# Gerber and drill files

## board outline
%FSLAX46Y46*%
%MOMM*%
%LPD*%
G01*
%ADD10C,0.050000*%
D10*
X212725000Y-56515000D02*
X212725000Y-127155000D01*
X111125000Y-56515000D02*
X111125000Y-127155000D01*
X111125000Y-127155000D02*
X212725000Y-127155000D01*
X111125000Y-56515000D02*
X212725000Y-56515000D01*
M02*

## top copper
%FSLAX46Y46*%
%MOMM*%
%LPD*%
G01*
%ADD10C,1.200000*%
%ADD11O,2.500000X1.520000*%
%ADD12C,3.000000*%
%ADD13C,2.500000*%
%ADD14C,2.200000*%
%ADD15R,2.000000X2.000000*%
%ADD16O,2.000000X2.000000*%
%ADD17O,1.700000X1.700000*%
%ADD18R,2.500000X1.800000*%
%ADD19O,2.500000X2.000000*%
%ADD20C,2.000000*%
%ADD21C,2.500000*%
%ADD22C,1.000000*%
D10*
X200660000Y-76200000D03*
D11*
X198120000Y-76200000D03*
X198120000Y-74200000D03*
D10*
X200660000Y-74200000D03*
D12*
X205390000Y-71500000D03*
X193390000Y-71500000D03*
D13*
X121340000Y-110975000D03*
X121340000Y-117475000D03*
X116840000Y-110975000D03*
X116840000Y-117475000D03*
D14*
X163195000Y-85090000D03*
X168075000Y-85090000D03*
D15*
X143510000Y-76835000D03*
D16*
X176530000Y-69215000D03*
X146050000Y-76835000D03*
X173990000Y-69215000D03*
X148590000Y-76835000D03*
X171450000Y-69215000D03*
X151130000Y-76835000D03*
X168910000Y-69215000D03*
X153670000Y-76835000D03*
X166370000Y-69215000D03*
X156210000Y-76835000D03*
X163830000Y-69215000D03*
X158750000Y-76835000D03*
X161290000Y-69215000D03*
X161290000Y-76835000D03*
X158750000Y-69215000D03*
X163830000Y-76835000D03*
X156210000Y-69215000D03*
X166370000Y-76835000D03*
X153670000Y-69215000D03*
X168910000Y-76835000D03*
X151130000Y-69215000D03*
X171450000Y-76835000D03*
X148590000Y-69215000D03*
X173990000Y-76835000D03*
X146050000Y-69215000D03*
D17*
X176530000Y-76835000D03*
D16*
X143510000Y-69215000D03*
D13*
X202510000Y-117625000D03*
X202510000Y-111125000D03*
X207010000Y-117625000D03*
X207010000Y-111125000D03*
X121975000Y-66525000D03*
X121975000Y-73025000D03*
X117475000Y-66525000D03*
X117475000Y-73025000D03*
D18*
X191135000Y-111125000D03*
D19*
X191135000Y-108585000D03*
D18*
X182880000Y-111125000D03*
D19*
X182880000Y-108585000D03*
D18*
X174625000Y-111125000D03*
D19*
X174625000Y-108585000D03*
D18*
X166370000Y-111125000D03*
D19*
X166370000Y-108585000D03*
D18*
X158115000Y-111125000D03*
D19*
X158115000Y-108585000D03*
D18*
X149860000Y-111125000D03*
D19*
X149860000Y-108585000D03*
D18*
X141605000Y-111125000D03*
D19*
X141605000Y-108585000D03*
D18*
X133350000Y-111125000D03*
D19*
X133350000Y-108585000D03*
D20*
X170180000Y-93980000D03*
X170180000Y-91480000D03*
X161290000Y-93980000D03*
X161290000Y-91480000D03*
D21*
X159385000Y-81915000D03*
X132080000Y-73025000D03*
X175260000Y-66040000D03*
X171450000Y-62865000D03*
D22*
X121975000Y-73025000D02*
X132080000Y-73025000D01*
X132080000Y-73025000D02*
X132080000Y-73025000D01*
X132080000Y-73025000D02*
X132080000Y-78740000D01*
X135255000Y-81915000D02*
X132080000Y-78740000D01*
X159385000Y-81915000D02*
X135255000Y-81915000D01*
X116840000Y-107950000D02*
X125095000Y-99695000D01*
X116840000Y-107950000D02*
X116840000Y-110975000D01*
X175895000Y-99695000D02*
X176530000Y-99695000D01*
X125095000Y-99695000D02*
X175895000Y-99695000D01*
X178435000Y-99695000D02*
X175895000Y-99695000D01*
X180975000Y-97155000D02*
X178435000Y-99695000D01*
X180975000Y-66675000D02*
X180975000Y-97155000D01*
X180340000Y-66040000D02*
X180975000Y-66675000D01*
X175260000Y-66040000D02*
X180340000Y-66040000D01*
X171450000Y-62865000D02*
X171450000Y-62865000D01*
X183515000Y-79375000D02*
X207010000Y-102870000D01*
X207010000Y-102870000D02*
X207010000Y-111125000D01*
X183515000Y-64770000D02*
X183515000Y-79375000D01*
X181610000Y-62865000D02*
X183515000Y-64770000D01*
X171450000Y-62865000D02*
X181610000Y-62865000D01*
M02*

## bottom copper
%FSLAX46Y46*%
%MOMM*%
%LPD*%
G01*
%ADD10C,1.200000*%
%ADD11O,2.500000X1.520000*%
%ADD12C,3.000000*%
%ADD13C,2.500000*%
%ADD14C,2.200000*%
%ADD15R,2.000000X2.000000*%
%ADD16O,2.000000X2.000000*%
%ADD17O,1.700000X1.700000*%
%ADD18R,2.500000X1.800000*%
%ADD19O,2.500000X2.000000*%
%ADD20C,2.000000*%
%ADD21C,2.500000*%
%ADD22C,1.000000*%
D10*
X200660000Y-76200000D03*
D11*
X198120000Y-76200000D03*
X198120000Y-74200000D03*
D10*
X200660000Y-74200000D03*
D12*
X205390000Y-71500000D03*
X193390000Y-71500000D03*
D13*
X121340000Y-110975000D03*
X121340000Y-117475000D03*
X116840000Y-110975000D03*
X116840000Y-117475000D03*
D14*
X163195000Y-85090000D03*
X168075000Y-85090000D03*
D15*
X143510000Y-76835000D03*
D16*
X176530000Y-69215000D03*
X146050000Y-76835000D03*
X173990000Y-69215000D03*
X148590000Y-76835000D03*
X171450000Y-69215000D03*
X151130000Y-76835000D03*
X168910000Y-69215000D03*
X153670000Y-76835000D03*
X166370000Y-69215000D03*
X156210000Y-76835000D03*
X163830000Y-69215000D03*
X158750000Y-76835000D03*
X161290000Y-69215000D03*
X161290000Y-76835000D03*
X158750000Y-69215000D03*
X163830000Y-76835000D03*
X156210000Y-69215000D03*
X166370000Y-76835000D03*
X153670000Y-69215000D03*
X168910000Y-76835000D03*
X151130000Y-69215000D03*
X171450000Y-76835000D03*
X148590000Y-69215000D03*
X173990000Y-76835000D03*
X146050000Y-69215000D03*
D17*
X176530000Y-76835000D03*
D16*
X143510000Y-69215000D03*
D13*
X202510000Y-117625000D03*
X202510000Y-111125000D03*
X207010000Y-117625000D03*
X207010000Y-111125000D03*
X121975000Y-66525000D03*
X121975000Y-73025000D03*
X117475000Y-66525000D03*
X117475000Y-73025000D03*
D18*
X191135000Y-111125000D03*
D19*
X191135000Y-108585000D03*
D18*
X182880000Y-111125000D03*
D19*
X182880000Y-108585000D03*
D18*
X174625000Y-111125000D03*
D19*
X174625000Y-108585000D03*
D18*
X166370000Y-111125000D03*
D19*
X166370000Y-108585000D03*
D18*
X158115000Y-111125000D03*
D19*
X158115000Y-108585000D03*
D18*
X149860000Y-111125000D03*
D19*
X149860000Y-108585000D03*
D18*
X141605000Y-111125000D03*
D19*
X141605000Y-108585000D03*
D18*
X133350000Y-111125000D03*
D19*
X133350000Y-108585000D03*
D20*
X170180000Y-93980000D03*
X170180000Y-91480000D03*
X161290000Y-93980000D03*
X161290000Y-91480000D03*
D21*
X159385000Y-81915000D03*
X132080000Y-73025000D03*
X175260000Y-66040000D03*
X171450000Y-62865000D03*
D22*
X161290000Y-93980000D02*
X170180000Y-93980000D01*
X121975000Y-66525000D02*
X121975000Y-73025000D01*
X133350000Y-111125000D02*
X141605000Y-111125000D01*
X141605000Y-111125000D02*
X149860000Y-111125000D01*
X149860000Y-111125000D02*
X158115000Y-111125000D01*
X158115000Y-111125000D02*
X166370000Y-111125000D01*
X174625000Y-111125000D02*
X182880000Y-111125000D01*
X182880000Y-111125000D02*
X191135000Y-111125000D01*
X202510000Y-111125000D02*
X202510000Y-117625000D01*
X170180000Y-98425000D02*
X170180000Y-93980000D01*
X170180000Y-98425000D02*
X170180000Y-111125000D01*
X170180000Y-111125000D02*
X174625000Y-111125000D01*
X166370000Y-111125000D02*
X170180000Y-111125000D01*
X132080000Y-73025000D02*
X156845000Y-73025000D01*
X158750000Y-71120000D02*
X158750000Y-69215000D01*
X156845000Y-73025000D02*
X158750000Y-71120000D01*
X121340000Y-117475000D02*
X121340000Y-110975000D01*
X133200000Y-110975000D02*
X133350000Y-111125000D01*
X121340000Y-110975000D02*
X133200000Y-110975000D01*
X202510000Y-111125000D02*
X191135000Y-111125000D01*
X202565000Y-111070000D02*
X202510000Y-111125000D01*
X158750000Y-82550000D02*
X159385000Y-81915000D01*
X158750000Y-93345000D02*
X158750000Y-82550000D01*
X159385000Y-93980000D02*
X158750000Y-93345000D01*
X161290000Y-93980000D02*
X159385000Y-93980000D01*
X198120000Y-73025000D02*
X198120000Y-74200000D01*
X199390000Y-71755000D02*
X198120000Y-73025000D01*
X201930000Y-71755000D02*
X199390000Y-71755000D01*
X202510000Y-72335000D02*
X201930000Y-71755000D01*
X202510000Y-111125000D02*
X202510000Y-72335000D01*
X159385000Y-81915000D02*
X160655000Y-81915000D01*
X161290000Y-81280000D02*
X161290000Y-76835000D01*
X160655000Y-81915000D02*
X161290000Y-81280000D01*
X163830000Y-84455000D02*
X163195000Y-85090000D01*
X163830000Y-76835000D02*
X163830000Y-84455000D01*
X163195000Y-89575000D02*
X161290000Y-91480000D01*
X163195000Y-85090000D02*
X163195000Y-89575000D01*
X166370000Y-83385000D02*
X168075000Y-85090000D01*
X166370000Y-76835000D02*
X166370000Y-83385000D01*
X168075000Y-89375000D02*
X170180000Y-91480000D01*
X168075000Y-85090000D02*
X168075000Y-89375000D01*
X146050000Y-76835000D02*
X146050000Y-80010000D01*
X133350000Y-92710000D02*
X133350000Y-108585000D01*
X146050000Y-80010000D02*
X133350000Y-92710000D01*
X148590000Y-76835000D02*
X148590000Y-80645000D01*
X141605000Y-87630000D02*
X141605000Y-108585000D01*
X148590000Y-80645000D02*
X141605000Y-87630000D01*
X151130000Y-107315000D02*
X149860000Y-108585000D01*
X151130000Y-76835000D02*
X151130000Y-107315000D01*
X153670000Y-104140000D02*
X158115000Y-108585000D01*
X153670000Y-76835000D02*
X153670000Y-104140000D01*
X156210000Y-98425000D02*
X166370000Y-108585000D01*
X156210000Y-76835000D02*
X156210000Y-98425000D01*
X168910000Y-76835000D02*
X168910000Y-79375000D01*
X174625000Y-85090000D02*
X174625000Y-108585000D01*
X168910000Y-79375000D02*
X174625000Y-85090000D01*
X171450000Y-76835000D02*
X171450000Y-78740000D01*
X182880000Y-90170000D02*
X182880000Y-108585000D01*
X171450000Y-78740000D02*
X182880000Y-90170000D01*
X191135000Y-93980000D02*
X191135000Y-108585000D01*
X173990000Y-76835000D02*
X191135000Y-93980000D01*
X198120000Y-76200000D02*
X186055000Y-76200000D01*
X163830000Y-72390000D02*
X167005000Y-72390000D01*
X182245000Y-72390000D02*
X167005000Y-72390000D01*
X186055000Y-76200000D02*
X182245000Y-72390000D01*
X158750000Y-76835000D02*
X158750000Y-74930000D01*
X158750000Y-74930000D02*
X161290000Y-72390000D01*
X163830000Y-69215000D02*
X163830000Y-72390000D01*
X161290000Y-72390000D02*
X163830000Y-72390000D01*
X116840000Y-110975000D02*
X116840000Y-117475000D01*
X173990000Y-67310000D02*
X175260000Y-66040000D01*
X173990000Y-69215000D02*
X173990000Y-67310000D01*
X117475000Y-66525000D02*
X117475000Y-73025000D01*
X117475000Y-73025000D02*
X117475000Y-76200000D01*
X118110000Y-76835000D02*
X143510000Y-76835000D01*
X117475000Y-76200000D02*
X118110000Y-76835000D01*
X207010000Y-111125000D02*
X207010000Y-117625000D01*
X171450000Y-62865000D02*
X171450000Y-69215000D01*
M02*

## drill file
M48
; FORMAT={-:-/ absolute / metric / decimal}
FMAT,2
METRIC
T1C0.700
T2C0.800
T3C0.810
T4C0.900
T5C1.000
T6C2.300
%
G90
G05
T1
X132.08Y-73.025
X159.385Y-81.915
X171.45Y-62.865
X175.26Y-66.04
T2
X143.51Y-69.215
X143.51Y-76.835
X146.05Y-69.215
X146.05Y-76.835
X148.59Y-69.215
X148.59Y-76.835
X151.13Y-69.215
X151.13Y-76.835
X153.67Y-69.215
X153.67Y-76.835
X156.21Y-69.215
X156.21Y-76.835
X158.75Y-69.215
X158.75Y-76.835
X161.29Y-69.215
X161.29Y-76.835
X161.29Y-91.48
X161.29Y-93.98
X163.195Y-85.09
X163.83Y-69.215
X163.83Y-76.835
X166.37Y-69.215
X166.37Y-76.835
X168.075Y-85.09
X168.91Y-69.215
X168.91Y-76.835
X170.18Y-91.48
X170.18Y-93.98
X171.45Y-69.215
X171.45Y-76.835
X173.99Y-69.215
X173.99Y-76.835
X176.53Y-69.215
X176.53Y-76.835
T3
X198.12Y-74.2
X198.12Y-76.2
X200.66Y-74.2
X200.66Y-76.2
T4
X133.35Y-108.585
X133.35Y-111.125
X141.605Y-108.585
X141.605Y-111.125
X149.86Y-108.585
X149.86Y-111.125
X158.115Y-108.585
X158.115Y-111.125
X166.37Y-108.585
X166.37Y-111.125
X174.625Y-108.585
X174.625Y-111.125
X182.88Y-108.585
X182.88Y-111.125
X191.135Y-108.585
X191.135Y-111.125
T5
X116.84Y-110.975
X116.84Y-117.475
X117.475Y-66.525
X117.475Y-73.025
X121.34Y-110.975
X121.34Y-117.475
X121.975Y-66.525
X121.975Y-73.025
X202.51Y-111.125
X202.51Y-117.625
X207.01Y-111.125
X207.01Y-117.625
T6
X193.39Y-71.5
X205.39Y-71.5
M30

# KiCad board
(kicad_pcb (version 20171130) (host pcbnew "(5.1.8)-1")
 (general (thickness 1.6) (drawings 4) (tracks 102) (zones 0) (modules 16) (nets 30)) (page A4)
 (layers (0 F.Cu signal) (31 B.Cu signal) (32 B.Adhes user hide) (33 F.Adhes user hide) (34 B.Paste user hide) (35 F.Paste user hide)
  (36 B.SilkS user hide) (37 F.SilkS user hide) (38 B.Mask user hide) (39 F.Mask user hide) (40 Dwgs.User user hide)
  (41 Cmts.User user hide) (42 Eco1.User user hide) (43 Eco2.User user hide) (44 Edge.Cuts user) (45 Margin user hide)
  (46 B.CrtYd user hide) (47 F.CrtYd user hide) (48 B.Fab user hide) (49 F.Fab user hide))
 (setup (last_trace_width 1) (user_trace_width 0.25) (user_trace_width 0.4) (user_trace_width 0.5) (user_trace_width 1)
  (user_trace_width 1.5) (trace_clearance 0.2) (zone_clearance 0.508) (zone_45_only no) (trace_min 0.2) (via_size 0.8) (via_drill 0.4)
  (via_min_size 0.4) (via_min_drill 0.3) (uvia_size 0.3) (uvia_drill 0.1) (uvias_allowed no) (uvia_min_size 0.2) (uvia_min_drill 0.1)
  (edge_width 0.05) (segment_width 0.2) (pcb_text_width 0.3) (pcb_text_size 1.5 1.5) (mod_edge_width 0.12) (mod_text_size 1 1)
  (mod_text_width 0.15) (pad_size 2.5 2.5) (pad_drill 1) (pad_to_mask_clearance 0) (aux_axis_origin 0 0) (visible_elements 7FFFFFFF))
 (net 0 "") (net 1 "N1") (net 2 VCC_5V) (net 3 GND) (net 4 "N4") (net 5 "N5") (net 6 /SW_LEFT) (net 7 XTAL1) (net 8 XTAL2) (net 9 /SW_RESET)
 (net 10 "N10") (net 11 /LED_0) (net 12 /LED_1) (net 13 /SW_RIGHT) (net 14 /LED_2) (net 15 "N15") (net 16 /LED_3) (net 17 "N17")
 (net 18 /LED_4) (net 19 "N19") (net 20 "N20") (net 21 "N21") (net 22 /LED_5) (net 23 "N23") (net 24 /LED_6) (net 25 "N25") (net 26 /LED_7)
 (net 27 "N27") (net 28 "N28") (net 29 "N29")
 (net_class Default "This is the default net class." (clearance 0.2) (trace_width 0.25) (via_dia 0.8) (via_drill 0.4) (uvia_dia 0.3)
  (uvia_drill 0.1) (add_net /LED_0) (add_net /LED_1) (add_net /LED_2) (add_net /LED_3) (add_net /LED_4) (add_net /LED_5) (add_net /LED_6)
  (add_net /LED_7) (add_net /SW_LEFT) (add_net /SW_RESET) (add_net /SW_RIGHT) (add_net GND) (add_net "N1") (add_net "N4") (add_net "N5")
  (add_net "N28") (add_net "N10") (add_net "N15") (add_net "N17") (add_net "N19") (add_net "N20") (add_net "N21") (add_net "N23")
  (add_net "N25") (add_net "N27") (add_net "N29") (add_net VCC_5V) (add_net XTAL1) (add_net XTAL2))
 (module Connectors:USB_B (layer F.Cu) (at 198.12 76.2 90)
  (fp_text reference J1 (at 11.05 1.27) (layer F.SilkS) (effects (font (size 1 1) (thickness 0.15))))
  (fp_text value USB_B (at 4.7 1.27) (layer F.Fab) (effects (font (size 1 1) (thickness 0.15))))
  (pad 2 thru_hole circle (at 0 2.54) (size 1.2 1.2) (drill 0.81) (layers *.Cu *.Mask) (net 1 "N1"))
  (pad 1 thru_hole oval (at 0 0) (size 2.5 1.52) (drill 0.81) (layers *.Cu *.Mask) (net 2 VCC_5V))
  (pad 4 thru_hole oval (at 2 0) (size 2.5 1.52) (drill 0.81) (layers *.Cu *.Mask) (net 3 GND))
  (pad 3 thru_hole circle (at 2 2.54) (size 1.2 1.2) (drill 0.81) (layers *.Cu *.Mask) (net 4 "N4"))
  (pad 5 thru_hole circle (at 4.7 7.27) (size 3 3) (drill 2.3) (layers *.Cu *.Mask) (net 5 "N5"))
  (pad 5 thru_hole circle (at 4.7 -4.73) (size 3 3) (drill 2.3) (layers *.Cu *.Mask) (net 5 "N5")))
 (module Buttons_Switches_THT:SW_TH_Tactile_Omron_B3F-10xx (layer F.Cu) (at 116.84 117.475 90)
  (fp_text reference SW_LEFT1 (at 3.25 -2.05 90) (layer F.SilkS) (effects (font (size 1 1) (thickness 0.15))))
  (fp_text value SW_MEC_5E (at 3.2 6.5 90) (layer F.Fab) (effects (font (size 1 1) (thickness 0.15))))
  (pad 4 thru_hole circle (at 6.5 4.5 90) (size 2.5 2.5) (drill 1) (layers *.Cu *.Mask) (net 3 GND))
  (pad 3 thru_hole circle (at 0 4.5 90) (size 2.5 2.5) (drill 1) (layers *.Cu *.Mask) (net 3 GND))
  (pad 2 thru_hole circle (at 6.5 0 90) (size 2.5 2.5) (drill 1) (layers *.Cu *.Mask) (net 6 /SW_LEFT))
  (pad 1 thru_hole circle (at 0 0 90) (size 2.5 2.5) (drill 1) (layers *.Cu *.Mask) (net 6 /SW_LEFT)))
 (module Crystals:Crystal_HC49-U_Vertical (layer F.Cu) (at 163.195 85.09)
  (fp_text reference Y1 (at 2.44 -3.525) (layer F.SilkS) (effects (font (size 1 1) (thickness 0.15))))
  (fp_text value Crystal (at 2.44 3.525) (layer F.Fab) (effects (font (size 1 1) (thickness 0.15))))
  (pad 1 thru_hole circle (at 0 0) (size 2.2 2.2) (drill 0.8) (layers *.Cu *.Mask) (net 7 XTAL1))
  (pad 2 thru_hole circle (at 4.88 0) (size 2.2 2.2) (drill 0.8) (layers *.Cu *.Mask) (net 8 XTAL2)))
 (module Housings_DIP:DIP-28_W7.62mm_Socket (layer F.Cu) (at 143.51 76.835 90)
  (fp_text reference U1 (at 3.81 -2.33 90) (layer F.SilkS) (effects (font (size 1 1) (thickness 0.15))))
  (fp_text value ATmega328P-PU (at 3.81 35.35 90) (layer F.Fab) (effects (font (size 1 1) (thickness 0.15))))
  (pad 1 thru_hole rect (at 0 0 90) (size 2 2) (drill 0.8) (layers *.Cu *.Mask) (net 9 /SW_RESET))
  (pad 15 thru_hole oval (at 7.62 33.02 90) (size 2 2) (drill 0.8) (layers *.Cu *.Mask) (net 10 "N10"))
  (pad 2 thru_hole oval (at 0 2.54 90) (size 2 2) (drill 0.8) (layers *.Cu *.Mask) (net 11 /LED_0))
  (pad 16 thru_hole oval (at 7.62 30.48 90) (size 2 2) (drill 0.8) (layers *.Cu *.Mask) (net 6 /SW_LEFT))
  (pad 3 thru_hole oval (at 0 5.08 90) (size 2 2) (drill 0.8) (layers *.Cu *.Mask) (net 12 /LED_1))
  (pad 17 thru_hole oval (at 7.62 27.94 90) (size 2 2) (drill 0.8) (layers *.Cu *.Mask) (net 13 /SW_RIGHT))
  (pad 4 thru_hole oval (at 0 7.62 90) (size 2 2) (drill 0.8) (layers *.Cu *.Mask) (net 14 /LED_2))
  (pad 18 thru_hole oval (at 7.62 25.4 90) (size 2 2) (drill 0.8) (layers *.Cu *.Mask) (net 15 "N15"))
  (pad 5 thru_hole oval (at 0 10.16 90) (size 2 2) (drill 0.8) (layers *.Cu *.Mask) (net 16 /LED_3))
  (pad 19 thru_hole oval (at 7.62 22.86 90) (size 2 2) (drill 0.8) (layers *.Cu *.Mask) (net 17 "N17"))
  (pad 6 thru_hole oval (at 0 12.7 90) (size 2 2) (drill 0.8) (layers *.Cu *.Mask) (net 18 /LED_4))
  (pad 20 thru_hole oval (at 7.62 20.32 90) (size 2 2) (drill 0.8) (layers *.Cu *.Mask) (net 2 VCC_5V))
  (pad 7 thru_hole oval (at 0 15.24 90) (size 2 2) (drill 0.8) (layers *.Cu *.Mask) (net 2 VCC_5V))
  (pad 21 thru_hole oval (at 7.62 17.78 90) (size 2 2) (drill 0.8) (layers *.Cu *.Mask) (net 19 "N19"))
  (pad 8 thru_hole oval (at 0 17.78 90) (size 2 2) (drill 0.8) (layers *.Cu *.Mask) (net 3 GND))
  (pad 22 thru_hole oval (at 7.62 15.24 90) (size 2 2) (drill 0.8) (layers *.Cu *.Mask) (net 3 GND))
  (pad 9 thru_hole oval (at 0 20.32 90) (size 2 2) (drill 0.8) (layers *.Cu *.Mask) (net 7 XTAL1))
  (pad 23 thru_hole oval (at 7.62 12.7 90) (size 2 2) (drill 0.8) (layers *.Cu *.Mask) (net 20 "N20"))
  (pad 10 thru_hole oval (at 0 22.86 90) (size 2 2) (drill 0.8) (layers *.Cu *.Mask) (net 8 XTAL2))
  (pad 24 thru_hole oval (at 7.62 10.16 90) (size 2 2) (drill 0.8) (layers *.Cu *.Mask) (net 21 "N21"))
  (pad 11 thru_hole oval (at 0 25.4 90) (size 2 2) (drill 0.8) (layers *.Cu *.Mask) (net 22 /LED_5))
  (pad 25 thru_hole oval (at 7.62 7.62 90) (size 2 2) (drill 0.8) (layers *.Cu *.Mask) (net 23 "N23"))
  (pad 12 thru_hole oval (at 0 27.94 90) (size 2 2) (drill 0.8) (layers *.Cu *.Mask) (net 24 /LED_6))
  (pad 26 thru_hole oval (at 7.62 5.08 90) (size 2 2) (drill 0.8) (layers *.Cu *.Mask) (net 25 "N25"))
  (pad 13 thru_hole oval (at 0 30.48 90) (size 2 2) (drill 0.8) (layers *.Cu *.Mask) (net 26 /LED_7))
  (pad 27 thru_hole oval (at 7.62 2.54 90) (size 2 2) (drill 0.8) (layers *.Cu *.Mask) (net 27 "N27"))
  (pad 14 thru_hole oval (at 0 33.02 90) (size 1.7 1.7) (drill 0.8) (layers *.Cu *.Mask) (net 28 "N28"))
  (pad 28 thru_hole oval (at 7.62 0 90) (size 2 2) (drill 0.8) (layers *.Cu *.Mask) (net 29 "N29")))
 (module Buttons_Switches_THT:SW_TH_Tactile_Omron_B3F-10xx (layer F.Cu) (at 207.01 111.125 270)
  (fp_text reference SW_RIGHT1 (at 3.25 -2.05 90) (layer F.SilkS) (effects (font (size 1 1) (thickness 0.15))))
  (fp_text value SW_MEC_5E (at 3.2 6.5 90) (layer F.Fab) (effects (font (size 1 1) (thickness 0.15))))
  (pad 4 thru_hole circle (at 6.5 4.5 270) (size 2.5 2.5) (drill 1) (layers *.Cu *.Mask) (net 3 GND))
  (pad 3 thru_hole circle (at 0 4.5 270) (size 2.5 2.5) (drill 1) (layers *.Cu *.Mask) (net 3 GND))
  (pad 2 thru_hole circle (at 6.5 0 270) (size 2.5 2.5) (drill 1) (layers *.Cu *.Mask) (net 13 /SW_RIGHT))
  (pad 1 thru_hole circle (at 0 0 270) (size 2.5 2.5) (drill 1) (layers *.Cu *.Mask) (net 13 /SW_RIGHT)))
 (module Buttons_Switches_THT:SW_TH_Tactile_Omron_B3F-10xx (layer F.Cu) (at 117.475 73.025 90)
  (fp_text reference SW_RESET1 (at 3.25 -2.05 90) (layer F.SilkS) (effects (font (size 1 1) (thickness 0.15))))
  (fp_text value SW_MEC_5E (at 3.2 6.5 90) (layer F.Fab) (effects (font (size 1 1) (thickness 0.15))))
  (pad 4 thru_hole circle (at 6.5 4.5 90) (size 2.5 2.5) (drill 1) (layers *.Cu *.Mask) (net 3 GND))
  (pad 3 thru_hole circle (at 0 4.5 90) (size 2.5 2.5) (drill 1) (layers *.Cu *.Mask) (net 3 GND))
  (pad 2 thru_hole circle (at 6.5 0 90) (size 2.5 2.5) (drill 1) (layers *.Cu *.Mask) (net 9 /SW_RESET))
  (pad 1 thru_hole circle (at 0 0 90) (size 2.5 2.5) (drill 1) (layers *.Cu *.Mask) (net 9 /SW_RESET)))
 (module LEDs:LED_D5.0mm (layer F.Cu) (at 191.135 111.125 90)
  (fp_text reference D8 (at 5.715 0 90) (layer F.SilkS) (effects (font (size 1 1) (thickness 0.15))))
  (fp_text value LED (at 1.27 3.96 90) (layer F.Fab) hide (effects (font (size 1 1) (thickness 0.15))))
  (pad 1 thru_hole rect (at 0 0 90) (size 1.8 2.5) (drill 0.9) (layers *.Cu *.Mask) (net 3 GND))
  (pad 2 thru_hole oval (at 2.54 0 90) (size 2 2.5) (drill 0.9) (layers *.Cu *.Mask) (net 26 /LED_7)))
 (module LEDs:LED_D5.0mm (layer F.Cu) (at 182.88 111.125 90)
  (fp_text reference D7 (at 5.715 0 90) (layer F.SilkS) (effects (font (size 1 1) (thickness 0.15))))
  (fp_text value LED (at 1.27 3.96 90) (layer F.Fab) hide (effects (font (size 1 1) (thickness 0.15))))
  (pad 1 thru_hole rect (at 0 0 90) (size 1.8 2.5) (drill 0.9) (layers *.Cu *.Mask) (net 3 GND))
  (pad 2 thru_hole oval (at 2.54 0 90) (size 2 2.5) (drill 0.9) (layers *.Cu *.Mask) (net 24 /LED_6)))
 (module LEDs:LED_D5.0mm (layer F.Cu) (at 174.625 111.125 90)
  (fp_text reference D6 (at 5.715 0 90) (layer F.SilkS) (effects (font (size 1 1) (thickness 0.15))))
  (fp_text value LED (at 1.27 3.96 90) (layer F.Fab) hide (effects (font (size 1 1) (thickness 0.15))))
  (pad 1 thru_hole rect (at 0 0 90) (size 1.8 2.5) (drill 0.9) (layers *.Cu *.Mask) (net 3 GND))
  (pad 2 thru_hole oval (at 2.54 0 90) (size 2 2.5) (drill 0.9) (layers *.Cu *.Mask) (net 22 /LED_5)))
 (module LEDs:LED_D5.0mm (layer F.Cu) (at 166.37 111.125 90)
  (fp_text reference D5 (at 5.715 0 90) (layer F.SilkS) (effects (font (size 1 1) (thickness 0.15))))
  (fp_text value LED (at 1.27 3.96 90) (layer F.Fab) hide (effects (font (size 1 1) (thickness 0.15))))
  (pad 1 thru_hole rect (at 0 0 90) (size 1.8 2.5) (drill 0.9) (layers *.Cu *.Mask) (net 3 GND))
  (pad 2 thru_hole oval (at 2.54 0 90) (size 2 2.5) (drill 0.9) (layers *.Cu *.Mask) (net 18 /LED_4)))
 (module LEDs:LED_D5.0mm (layer F.Cu) (at 158.115 111.125 90)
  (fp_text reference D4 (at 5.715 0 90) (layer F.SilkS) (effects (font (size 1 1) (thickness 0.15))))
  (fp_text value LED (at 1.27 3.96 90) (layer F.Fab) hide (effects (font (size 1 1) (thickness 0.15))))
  (pad 1 thru_hole rect (at 0 0 90) (size 1.8 2.5) (drill 0.9) (layers *.Cu *.Mask) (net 3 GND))
  (pad 2 thru_hole oval (at 2.54 0 90) (size 2 2.5) (drill 0.9) (layers *.Cu *.Mask) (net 16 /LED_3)))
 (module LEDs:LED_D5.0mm (layer F.Cu) (at 149.86 111.125 90)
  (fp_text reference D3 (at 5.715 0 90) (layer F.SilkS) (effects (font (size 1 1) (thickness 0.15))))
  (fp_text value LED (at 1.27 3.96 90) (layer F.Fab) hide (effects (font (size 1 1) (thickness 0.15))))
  (pad 1 thru_hole rect (at 0 0 90) (size 1.8 2.5) (drill 0.9) (layers *.Cu *.Mask) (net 3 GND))
  (pad 2 thru_hole oval (at 2.54 0 90) (size 2 2.5) (drill 0.9) (layers *.Cu *.Mask) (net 14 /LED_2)))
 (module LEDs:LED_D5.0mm (layer F.Cu) (at 141.605 111.125 90)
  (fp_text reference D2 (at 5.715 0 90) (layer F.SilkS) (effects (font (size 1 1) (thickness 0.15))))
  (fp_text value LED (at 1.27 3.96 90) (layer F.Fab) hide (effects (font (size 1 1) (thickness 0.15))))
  (pad 1 thru_hole rect (at 0 0 90) (size 1.8 2.5) (drill 0.9) (layers *.Cu *.Mask) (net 3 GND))
  (pad 2 thru_hole oval (at 2.54 0 90) (size 2 2.5) (drill 0.9) (layers *.Cu *.Mask) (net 12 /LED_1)))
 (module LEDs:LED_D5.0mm (layer F.Cu) (at 133.35 111.125 90)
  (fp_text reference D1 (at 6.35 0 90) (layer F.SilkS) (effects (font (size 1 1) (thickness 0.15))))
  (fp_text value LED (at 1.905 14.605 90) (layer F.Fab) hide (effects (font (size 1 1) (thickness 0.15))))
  (pad 1 thru_hole rect (at 0 0 90) (size 1.8 2.5) (drill 0.9) (layers *.Cu *.Mask) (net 3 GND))
  (pad 2 thru_hole oval (at 2.54 0 90) (size 2 2.5) (drill 0.9) (layers *.Cu *.Mask) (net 11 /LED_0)))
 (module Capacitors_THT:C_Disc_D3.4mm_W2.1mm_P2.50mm (layer F.Cu) (at 170.18 93.98 90)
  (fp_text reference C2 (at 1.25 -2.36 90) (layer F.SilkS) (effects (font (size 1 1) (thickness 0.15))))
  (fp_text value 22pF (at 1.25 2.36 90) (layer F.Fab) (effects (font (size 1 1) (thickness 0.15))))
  (pad 1 thru_hole circle (at 0 0 90) (size 2 2) (drill 0.8) (layers *.Cu *.Mask) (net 3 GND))
  (pad 2 thru_hole circle (at 2.5 0 90) (size 2 2) (drill 0.8) (layers *.Cu *.Mask) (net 8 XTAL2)))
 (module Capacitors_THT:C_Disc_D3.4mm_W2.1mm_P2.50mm (layer F.Cu) (at 161.29 93.98 90)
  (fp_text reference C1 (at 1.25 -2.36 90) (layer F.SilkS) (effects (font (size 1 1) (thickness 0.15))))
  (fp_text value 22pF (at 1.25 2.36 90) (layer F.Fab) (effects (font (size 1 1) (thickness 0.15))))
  (pad 1 thru_hole circle (at 0 0 90) (size 2 2) (drill 0.8) (layers *.Cu *.Mask) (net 3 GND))
  (pad 2 thru_hole circle (at 2.5 0 90) (size 2 2) (drill 0.8) (layers *.Cu *.Mask) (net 7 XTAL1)))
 (gr_line (start 212.725 56.515) (end 212.725 127.155) (layer Edge.Cuts) (width 0.05))
 (gr_line (start 111.125 56.515) (end 111.125 127.155) (layer Edge.Cuts) (width 0.05))
 (gr_line (start 111.125 127.155) (end 212.725 127.155) (layer Edge.Cuts) (width 0.05))
 (gr_line (start 111.125 56.515) (end 212.725 56.515) (layer Edge.Cuts) (width 0.05))
 (segment (start 161.29 93.98) (end 170.18 93.98) (width 1) (layer B.Cu) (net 3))
 (segment (start 121.975 66.525) (end 121.975 73.025) (width 1) (layer B.Cu) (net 3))
 (segment (start 133.35 111.125) (end 141.605 111.125) (width 1) (layer B.Cu) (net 3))
 (segment (start 141.605 111.125) (end 149.86 111.125) (width 1) (layer B.Cu) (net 3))
 (segment (start 149.86 111.125) (end 158.115 111.125) (width 1) (layer B.Cu) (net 3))
 (segment (start 158.115 111.125) (end 166.37 111.125) (width 1) (layer B.Cu) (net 3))
 (segment (start 174.625 111.125) (end 182.88 111.125) (width 1) (layer B.Cu) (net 3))
 (segment (start 182.88 111.125) (end 191.135 111.125) (width 1) (layer B.Cu) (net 3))
 (segment (start 202.51 111.125) (end 202.51 117.625) (width 1) (layer B.Cu) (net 3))
 (segment (start 170.18 98.425) (end 170.18 93.98) (width 1) (layer B.Cu) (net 3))
 (segment (start 170.18 98.425) (end 170.18 111.125) (width 1) (layer B.Cu) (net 3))
 (segment (start 170.18 111.125) (end 174.625 111.125) (width 1) (layer B.Cu) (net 3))
 (segment (start 166.37 111.125) (end 170.18 111.125) (width 1) (layer B.Cu) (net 3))
 (via (at 159.385 81.915) (size 2.5) (drill 0.7) (layers F.Cu B.Cu) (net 3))
 (segment (start 121.975 73.025) (end 132.08 73.025) (width 1) (layer F.Cu) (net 3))
 (segment (start 132.08 73.025) (end 132.08 73.025) (width 1) (layer F.Cu) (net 3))
 (via (at 132.08 73.025) (size 2.5) (drill 0.7) (layers F.Cu B.Cu) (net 3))
 (segment (start 132.08 73.025) (end 156.845 73.025) (width 1) (layer B.Cu) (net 3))
 (segment (start 158.75 71.12) (end 158.75 69.215) (width 1) (layer B.Cu) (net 3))
 (segment (start 156.845 73.025) (end 158.75 71.12) (width 1) (layer B.Cu) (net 3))
 (segment (start 121.34 117.475) (end 121.34 110.975) (width 1) (layer B.Cu) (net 3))
 (segment (start 133.2 110.975) (end 133.35 111.125) (width 1) (layer B.Cu) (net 3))
 (segment (start 121.34 110.975) (end 133.2 110.975) (width 1) (layer B.Cu) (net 3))
 (segment (start 202.51 111.125) (end 191.135 111.125) (width 1) (layer B.Cu) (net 3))
 (segment (start 202.565 111.07) (end 202.51 111.125) (width 1) (layer B.Cu) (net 3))
 (segment (start 132.08 73.025) (end 132.08 78.74) (width 1) (layer F.Cu) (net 3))
 (segment (start 158.75 82.55) (end 159.385 81.915) (width 1) (layer B.Cu) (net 3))
 (segment (start 158.75 93.345) (end 158.75 82.55) (width 1) (layer B.Cu) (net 3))
 (segment (start 159.385 93.98) (end 158.75 93.345) (width 1) (layer B.Cu) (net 3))
 (segment (start 161.29 93.98) (end 159.385 93.98) (width 1) (layer B.Cu) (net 3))
 (segment (start 198.12 73.025) (end 198.12 74.2) (width 1) (layer B.Cu) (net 3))
 (segment (start 199.39 71.755) (end 198.12 73.025) (width 1) (layer B.Cu) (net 3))
 (segment (start 201.93 71.755) (end 199.39 71.755) (width 1) (layer B.Cu) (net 3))
 (segment (start 202.51 72.335) (end 201.93 71.755) (width 1) (layer B.Cu) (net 3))
 (segment (start 202.51 111.125) (end 202.51 72.335) (width 1) (layer B.Cu) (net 3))
 (segment (start 135.255 81.915) (end 132.08 78.74) (width 1) (layer F.Cu) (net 3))
 (segment (start 159.385 81.915) (end 135.255 81.915) (width 1) (layer F.Cu) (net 3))
 (segment (start 159.385 81.915) (end 160.655 81.915) (width 1) (layer B.Cu) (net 3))
 (segment (start 161.29 81.28) (end 161.29 76.835) (width 1) (layer B.Cu) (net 3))
 (segment (start 160.655 81.915) (end 161.29 81.28) (width 1) (layer B.Cu) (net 3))
 (segment (start 163.83 84.455) (end 163.195 85.09) (width 1) (layer B.Cu) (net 7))
 (segment (start 163.83 76.835) (end 163.83 84.455) (width 1) (layer B.Cu) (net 7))
 (segment (start 163.195 89.575) (end 161.29 91.48) (width 1) (layer B.Cu) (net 7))
 (segment (start 163.195 85.09) (end 163.195 89.575) (width 1) (layer B.Cu) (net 7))
 (segment (start 166.37 83.385) (end 168.075 85.09) (width 1) (layer B.Cu) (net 8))
 (segment (start 166.37 76.835) (end 166.37 83.385) (width 1) (layer B.Cu) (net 8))
 (segment (start 168.075 89.375) (end 170.18 91.48) (width 1) (layer B.Cu) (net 8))
 (segment (start 168.075 85.09) (end 168.075 89.375) (width 1) (layer B.Cu) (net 8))
 (segment (start 146.05 76.835) (end 146.05 80.01) (width 1) (layer B.Cu) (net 11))
 (segment (start 133.35 92.71) (end 133.35 108.585) (width 1) (layer B.Cu) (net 11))
 (segment (start 146.05 80.01) (end 133.35 92.71) (width 1) (layer B.Cu) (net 11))
 (segment (start 148.59 76.835) (end 148.59 80.645) (width 1) (layer B.Cu) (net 12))
 (segment (start 141.605 87.63) (end 141.605 108.585) (width 1) (layer B.Cu) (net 12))
 (segment (start 148.59 80.645) (end 141.605 87.63) (width 1) (layer B.Cu) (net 12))
 (segment (start 151.13 107.315) (end 149.86 108.585) (width 1) (layer B.Cu) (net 14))
 (segment (start 151.13 76.835) (end 151.13 107.315) (width 1) (layer B.Cu) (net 14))
 (segment (start 153.67 104.14) (end 158.115 108.585) (width 1) (layer B.Cu) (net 16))
 (segment (start 153.67 76.835) (end 153.67 104.14) (width 1) (layer B.Cu) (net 16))
 (segment (start 156.21 98.425) (end 166.37 108.585) (width 1) (layer B.Cu) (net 18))
 (segment (start 156.21 76.835) (end 156.21 98.425) (width 1) (layer B.Cu) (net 18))
 (segment (start 168.91 76.835) (end 168.91 79.375) (width 1) (layer B.Cu) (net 22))
 (segment (start 174.625 85.09) (end 174.625 108.585) (width 1) (layer B.Cu) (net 22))
 (segment (start 168.91 79.375) (end 174.625 85.09) (width 1) (layer B.Cu) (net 22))
 (segment (start 171.45 76.835) (end 171.45 78.74) (width 1) (layer B.Cu) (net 24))
 (segment (start 182.88 90.17) (end 182.88 108.585) (width 1) (layer B.Cu) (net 24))
 (segment (start 171.45 78.74) (end 182.88 90.17) (width 1) (layer B.Cu) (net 24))
 (segment (start 191.135 93.98) (end 191.135 108.585) (width 1) (layer B.Cu) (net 26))
 (segment (start 173.99 76.835) (end 191.135 93.98) (width 1) (layer B.Cu) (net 26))
 (segment (start 198.12 76.2) (end 186.055 76.2) (width 1) (layer B.Cu) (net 2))
 (segment (start 163.83 72.39) (end 167.005 72.39) (width 1) (layer B.Cu) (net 2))
 (segment (start 182.245 72.39) (end 167.005 72.39) (width 1) (layer B.Cu) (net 2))
 (segment (start 186.055 76.2) (end 182.245 72.39) (width 1) (layer B.Cu) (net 2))
 (segment (start 158.75 76.835) (end 158.75 74.93) (width 1) (layer B.Cu) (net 2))
 (segment (start 158.75 74.93) (end 161.29 72.39) (width 1) (layer B.Cu) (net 2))
 (segment (start 163.83 69.215) (end 163.83 72.39) (width 1) (layer B.Cu) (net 2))
 (segment (start 161.29 72.39) (end 163.83 72.39) (width 1) (layer B.Cu) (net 2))
 (segment (start 116.84 110.975) (end 116.84 117.475) (width 1) (layer B.Cu) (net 6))
 (segment (start 116.84 107.95) (end 125.095 99.695) (width 1) (layer F.Cu) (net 6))
 (via (at 175.26 66.04) (size 2.5) (drill 0.7) (layers F.Cu B.Cu) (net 6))
 (segment (start 116.84 107.95) (end 116.84 110.975) (width 1) (layer F.Cu) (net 6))
 (segment (start 173.99 67.31) (end 175.26 66.04) (width 1) (layer B.Cu) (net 6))
 (segment (start 173.99 69.215) (end 173.99 67.31) (width 1) (layer B.Cu) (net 6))
 (segment (start 175.895 99.695) (end 176.53 99.695) (width 1) (layer F.Cu) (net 6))
 (segment (start 125.095 99.695) (end 175.895 99.695) (width 1) (layer F.Cu) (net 6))
 (segment (start 178.435 99.695) (end 175.895 99.695) (width 1) (layer F.Cu) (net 6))
 (segment (start 180.975 97.155) (end 178.435 99.695) (width 1) (layer F.Cu) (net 6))
 (segment (start 180.975 66.675) (end 180.975 97.155) (width 1) (layer F.Cu) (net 6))
 (segment (start 180.34 66.04) (end 180.975 66.675) (width 1) (layer F.Cu) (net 6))
 (segment (start 175.26 66.04) (end 180.34 66.04) (width 1) (layer F.Cu) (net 6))
 (segment (start 117.475 66.525) (end 117.475 73.025) (width 1) (layer B.Cu) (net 9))
 (segment (start 117.475 73.025) (end 117.475 76.2) (width 1) (layer B.Cu) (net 9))
 (segment (start 118.11 76.835) (end 143.51 76.835) (width 1) (layer B.Cu) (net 9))
 (segment (start 117.475 76.2) (end 118.11 76.835) (width 1) (layer B.Cu) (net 9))
 (segment (start 207.01 111.125) (end 207.01 117.625) (width 1) (layer B.Cu) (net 13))
 (segment (start 171.45 62.865) (end 171.45 62.865) (width 1) (layer F.Cu) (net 13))
 (via (at 171.45 62.865) (size 2.5) (drill 0.7) (layers F.Cu B.Cu) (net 13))
 (segment (start 171.45 62.865) (end 171.45 69.215) (width 1) (layer B.Cu) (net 13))
 (segment (start 183.515 79.375) (end 207.01 102.87) (width 1) (layer F.Cu) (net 13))
 (segment (start 207.01 102.87) (end 207.01 111.125) (width 1) (layer F.Cu) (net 13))
 (segment (start 183.515 64.77) (end 183.515 79.375) (width 1) (layer F.Cu) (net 13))
 (segment (start 181.61 62.865) (end 183.515 64.77) (width 1) (layer F.Cu) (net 13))
 (segment (start 171.45 62.865) (end 181.61 62.865) (width 1) (layer F.Cu) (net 13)))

